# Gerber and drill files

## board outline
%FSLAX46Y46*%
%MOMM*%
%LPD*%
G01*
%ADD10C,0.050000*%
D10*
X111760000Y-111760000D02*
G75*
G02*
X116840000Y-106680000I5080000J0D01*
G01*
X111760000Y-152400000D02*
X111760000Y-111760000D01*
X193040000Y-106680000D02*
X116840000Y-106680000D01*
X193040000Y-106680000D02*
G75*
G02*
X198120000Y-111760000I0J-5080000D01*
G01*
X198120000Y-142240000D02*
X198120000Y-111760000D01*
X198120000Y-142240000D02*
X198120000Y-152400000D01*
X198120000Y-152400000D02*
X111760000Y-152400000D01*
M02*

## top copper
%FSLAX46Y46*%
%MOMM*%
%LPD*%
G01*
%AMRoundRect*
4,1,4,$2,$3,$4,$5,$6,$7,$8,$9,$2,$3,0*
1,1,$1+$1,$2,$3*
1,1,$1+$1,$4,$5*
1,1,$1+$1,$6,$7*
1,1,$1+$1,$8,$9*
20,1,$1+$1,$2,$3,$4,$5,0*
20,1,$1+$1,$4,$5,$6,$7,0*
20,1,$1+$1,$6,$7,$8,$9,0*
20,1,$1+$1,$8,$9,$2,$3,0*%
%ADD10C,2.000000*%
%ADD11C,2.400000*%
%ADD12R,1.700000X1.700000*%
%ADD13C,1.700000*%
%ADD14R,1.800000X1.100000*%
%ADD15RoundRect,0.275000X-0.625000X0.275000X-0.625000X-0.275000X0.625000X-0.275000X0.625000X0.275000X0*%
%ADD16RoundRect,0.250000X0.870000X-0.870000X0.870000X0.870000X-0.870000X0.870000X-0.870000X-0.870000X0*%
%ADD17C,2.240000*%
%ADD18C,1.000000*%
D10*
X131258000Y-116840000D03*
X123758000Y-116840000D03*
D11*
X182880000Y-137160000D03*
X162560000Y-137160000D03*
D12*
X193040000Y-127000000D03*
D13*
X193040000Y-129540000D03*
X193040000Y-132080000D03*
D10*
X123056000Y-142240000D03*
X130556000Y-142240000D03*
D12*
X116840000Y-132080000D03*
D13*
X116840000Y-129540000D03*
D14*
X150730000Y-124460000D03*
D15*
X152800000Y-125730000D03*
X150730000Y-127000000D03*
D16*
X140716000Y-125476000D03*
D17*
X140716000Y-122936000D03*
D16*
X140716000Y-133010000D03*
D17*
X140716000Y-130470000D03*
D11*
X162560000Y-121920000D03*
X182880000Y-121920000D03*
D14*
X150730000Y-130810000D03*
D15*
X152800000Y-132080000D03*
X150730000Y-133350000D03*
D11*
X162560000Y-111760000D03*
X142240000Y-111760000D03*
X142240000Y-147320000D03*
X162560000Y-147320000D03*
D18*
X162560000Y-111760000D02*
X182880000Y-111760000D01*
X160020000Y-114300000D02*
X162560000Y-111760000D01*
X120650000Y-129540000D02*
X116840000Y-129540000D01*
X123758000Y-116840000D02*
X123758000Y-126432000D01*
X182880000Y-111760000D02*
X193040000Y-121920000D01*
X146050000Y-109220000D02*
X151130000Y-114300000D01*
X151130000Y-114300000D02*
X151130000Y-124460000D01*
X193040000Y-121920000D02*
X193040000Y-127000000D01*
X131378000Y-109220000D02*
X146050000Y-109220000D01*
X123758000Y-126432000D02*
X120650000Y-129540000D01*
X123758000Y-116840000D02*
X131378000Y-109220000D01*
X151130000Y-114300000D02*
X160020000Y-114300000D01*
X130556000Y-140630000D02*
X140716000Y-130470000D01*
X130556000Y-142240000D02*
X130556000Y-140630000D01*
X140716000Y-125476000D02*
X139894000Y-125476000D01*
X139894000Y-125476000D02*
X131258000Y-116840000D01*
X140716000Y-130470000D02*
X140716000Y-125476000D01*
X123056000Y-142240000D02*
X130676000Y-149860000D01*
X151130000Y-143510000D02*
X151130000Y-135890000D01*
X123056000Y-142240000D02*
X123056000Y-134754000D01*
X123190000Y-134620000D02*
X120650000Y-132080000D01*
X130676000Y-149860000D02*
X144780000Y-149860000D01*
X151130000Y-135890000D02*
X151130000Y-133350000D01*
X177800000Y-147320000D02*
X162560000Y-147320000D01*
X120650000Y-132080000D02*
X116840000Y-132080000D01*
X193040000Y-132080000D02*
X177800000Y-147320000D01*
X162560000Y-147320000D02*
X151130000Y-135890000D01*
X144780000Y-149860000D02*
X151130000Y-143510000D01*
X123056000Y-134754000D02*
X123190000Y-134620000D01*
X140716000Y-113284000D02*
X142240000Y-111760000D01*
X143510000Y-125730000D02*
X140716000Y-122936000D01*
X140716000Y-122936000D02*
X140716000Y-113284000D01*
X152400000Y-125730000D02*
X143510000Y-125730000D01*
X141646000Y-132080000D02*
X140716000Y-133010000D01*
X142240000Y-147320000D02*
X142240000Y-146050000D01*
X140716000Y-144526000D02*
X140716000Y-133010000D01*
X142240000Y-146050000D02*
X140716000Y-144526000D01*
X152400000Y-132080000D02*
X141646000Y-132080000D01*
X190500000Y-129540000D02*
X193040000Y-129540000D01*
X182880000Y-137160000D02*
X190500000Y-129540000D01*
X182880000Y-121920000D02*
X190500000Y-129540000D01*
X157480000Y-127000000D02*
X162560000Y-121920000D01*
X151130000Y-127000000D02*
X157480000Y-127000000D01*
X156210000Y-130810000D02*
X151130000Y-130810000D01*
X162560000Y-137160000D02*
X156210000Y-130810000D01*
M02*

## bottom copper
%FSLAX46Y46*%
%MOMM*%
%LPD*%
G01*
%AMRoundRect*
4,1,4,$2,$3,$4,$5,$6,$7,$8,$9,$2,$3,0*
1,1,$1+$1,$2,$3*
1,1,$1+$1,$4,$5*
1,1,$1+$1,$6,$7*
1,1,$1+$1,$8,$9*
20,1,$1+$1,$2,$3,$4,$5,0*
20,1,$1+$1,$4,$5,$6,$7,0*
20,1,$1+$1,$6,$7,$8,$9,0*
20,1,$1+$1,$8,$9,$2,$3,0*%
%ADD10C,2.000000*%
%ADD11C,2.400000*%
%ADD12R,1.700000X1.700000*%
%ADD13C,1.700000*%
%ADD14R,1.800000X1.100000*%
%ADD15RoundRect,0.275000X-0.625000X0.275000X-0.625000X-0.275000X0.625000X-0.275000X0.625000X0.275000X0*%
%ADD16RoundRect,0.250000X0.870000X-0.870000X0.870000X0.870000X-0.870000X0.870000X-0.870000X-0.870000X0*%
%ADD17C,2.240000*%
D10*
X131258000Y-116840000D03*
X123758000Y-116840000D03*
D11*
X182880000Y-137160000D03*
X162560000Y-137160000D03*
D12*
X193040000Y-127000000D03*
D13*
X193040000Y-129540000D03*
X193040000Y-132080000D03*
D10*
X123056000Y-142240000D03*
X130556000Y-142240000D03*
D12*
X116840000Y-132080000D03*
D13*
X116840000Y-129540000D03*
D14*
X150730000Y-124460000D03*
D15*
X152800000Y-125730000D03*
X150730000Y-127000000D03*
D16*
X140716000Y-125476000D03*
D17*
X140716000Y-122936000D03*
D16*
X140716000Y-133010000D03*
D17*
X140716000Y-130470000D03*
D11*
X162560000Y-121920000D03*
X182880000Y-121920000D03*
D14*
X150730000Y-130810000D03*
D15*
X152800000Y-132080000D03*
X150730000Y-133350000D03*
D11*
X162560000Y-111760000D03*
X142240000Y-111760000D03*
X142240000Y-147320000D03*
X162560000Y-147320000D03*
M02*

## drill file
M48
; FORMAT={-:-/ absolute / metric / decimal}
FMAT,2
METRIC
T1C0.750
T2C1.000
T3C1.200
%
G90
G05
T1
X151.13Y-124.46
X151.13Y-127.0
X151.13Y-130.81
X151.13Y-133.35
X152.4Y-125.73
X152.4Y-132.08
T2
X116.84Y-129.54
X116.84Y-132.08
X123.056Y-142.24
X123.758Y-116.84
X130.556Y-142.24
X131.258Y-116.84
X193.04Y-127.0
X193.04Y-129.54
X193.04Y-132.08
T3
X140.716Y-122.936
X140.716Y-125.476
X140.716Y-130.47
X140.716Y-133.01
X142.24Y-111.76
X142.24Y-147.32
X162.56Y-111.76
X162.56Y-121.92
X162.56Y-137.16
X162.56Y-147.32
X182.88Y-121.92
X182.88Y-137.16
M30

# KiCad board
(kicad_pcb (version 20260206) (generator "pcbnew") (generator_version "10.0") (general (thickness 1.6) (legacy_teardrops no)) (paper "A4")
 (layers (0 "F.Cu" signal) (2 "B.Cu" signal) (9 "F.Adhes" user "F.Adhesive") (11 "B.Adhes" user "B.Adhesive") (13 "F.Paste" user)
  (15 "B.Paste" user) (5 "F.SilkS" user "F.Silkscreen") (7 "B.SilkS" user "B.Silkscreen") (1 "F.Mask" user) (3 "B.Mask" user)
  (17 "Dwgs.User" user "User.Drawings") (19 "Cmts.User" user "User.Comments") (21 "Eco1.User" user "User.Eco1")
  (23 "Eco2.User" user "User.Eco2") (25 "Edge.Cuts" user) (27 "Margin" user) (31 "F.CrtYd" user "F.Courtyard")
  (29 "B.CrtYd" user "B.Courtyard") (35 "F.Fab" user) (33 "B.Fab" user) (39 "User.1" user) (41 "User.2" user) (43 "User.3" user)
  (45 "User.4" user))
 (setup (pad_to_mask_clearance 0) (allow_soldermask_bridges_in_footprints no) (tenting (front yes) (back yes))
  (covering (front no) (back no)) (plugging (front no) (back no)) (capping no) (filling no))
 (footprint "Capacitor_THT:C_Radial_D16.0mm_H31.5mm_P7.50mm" (layer "F.Cu") (at 131.258 116.84 180)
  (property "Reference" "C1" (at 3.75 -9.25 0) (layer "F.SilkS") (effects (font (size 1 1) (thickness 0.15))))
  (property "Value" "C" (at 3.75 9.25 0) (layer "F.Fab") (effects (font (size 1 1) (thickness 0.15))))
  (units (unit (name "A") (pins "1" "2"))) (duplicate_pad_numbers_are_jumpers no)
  (pad "1" thru_hole circle (at 0 0 180) (size 2 2) (drill 1) (layers "*.Cu" "*.Mask") (remove_unused_layers no) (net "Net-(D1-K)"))
  (pad "2" thru_hole circle (at 7.5 0 180) (size 2 2) (drill 1) (layers "*.Cu" "*.Mask") (remove_unused_layers no) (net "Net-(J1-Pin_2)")))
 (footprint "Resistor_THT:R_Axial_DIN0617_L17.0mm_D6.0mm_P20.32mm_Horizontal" (layer "F.Cu") (at 182.88 137.16 180)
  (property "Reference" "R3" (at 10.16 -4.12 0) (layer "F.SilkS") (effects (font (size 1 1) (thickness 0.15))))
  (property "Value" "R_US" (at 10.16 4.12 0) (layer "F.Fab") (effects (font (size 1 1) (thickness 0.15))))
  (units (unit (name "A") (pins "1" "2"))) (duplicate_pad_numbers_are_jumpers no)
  (pad "1" thru_hole circle (at 0 0 180) (size 2.4 2.4) (drill 1.2) (layers "*.Cu" "*.Mask") (remove_unused_layers no)
   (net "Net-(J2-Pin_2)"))
  (pad "2" thru_hole circle (at 20.32 0 180) (size 2.4 2.4) (drill 1.2) (layers "*.Cu" "*.Mask") (remove_unused_layers no)
   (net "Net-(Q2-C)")))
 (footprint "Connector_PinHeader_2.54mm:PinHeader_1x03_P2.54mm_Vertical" (layer "F.Cu") (at 193.04 127)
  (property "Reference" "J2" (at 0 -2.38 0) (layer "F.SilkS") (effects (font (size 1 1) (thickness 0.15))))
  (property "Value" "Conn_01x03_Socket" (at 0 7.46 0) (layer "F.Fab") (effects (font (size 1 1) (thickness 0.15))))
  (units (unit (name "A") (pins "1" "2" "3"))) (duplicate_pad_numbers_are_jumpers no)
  (pad "1" thru_hole rect (at 0 0) (size 1.7 1.7) (drill 1) (layers "*.Cu" "*.Mask") (remove_unused_layers no) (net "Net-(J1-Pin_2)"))
  (pad "2" thru_hole circle (at 0 2.54) (size 1.7 1.7) (drill 1) (layers "*.Cu" "*.Mask") (remove_unused_layers no) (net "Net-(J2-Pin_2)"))
  (pad "3" thru_hole circle (at 0 5.08) (size 1.7 1.7) (drill 1) (layers "*.Cu" "*.Mask") (remove_unused_layers no) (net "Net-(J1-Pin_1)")))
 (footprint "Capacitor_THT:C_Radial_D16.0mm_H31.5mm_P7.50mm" (layer "F.Cu") (at 123.056 142.24)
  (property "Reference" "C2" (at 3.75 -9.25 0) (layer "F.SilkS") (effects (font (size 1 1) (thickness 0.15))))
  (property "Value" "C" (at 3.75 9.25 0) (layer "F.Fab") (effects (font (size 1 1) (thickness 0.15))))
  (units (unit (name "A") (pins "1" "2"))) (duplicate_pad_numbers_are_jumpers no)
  (pad "1" thru_hole circle (at 0 0) (size 2 2) (drill 1) (layers "*.Cu" "*.Mask") (remove_unused_layers no) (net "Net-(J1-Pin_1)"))
  (pad "2" thru_hole circle (at 7.5 0) (size 2 2) (drill 1) (layers "*.Cu" "*.Mask") (remove_unused_layers no) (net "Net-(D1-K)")))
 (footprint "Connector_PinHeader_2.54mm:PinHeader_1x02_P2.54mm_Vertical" (layer "F.Cu") (at 116.84 132.08 180)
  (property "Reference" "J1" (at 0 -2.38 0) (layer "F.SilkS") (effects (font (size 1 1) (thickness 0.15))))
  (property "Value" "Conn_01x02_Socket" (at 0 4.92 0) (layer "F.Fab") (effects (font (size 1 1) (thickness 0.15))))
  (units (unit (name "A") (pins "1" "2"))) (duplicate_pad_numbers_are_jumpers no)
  (pad "1" thru_hole rect (at 0 0 180) (size 1.7 1.7) (drill 1) (layers "*.Cu" "*.Mask") (remove_unused_layers no) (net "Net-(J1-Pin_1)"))
  (pad "2" thru_hole circle (at 0 2.54 180) (size 1.7 1.7) (drill 1) (layers "*.Cu" "*.Mask") (remove_unused_layers no)
   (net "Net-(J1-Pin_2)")))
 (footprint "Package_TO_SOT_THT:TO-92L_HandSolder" (layer "F.Cu") (at 151.13 124.46 -90)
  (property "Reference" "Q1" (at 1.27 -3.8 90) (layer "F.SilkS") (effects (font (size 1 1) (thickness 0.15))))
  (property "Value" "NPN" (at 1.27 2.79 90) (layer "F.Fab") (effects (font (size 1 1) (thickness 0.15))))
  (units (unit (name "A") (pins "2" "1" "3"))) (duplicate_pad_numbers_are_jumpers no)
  (pad "1" thru_hole rect (at 0 0 270) (size 1.1 1.8) (drill 0.75 (offset 0 0.4)) (layers "*.Cu" "*.Mask") (remove_unused_layers no)
   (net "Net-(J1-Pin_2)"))
  (pad "2" thru_hole roundrect (at 1.27 -1.27 270) (size 1.1 1.8) (drill 0.75 (offset 0 -0.4)) (layers "*.Cu" "*.Mask")
   (remove_unused_layers no) (roundrect_rratio 0.25) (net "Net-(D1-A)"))
  (pad "3" thru_hole roundrect (at 2.54 0 270) (size 1.1 1.8) (drill 0.75 (offset 0 0.4)) (layers "*.Cu" "*.Mask") (remove_unused_layers no)
   (roundrect_rratio 0.25) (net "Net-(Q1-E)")))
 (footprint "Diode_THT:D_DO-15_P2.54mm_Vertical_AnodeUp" (layer "F.Cu") (at 140.716 125.476 90)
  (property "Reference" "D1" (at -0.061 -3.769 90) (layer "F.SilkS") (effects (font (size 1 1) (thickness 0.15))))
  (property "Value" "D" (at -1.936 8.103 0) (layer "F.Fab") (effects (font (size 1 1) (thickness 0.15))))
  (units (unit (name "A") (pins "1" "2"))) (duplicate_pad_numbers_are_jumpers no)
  (pad "1" thru_hole roundrect (at 0 0 90) (size 2.24 2.24) (drill 1.2) (layers "*.Cu" "*.Mask") (remove_unused_layers no)
   (roundrect_rratio 0.111607) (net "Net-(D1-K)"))
  (pad "2" thru_hole circle (at 2.54 0 90) (size 2.24 2.24) (drill 1.2) (layers "*.Cu" "*.Mask") (remove_unused_layers no)
   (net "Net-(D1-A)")))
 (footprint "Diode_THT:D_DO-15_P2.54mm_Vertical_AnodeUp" (layer "F.Cu") (at 140.716 133.01 90)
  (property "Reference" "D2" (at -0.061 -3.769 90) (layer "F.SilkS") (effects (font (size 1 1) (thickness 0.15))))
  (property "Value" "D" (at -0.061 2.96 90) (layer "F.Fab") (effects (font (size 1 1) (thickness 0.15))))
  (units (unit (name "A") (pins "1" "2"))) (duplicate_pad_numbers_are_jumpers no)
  (pad "1" thru_hole roundrect (at 0 0 90) (size 2.24 2.24) (drill 1.2) (layers "*.Cu" "*.Mask") (remove_unused_layers no)
   (roundrect_rratio 0.111607) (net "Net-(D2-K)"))
  (pad "2" thru_hole circle (at 2.54 0 90) (size 2.24 2.24) (drill 1.2) (layers "*.Cu" "*.Mask") (remove_unused_layers no)
   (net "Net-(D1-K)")))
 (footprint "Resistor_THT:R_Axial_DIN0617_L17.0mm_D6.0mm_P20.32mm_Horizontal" (layer "F.Cu") (at 162.56 121.92)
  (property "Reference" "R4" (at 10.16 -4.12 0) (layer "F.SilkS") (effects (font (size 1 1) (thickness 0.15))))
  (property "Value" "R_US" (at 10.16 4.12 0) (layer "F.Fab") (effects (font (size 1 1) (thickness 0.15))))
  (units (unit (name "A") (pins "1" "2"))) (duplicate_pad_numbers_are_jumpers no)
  (pad "1" thru_hole circle (at 0 0) (size 2.4 2.4) (drill 1.2) (layers "*.Cu" "*.Mask") (remove_unused_layers no) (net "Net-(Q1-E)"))
  (pad "2" thru_hole circle (at 20.32 0) (size 2.4 2.4) (drill 1.2) (layers "*.Cu" "*.Mask") (remove_unused_layers no)
   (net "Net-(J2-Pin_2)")))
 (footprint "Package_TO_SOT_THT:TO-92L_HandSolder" (layer "F.Cu") (at 151.13 130.81 -90)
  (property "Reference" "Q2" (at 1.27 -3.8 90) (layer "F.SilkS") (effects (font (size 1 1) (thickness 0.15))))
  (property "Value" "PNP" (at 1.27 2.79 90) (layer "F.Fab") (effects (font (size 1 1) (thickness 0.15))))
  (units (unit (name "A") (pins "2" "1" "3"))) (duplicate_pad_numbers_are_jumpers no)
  (pad "1" thru_hole rect (at 0 0 270) (size 1.1 1.8) (drill 0.75 (offset 0 0.4)) (layers "*.Cu" "*.Mask") (remove_unused_layers no)
   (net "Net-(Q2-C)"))
  (pad "2" thru_hole roundrect (at 1.27 -1.27 270) (size 1.1 1.8) (drill 0.75 (offset 0 -0.4)) (layers "*.Cu" "*.Mask")
   (remove_unused_layers no) (roundrect_rratio 0.25) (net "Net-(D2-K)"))
  (pad "3" thru_hole roundrect (at 2.54 0 270) (size 1.1 1.8) (drill 0.75 (offset 0 0.4)) (layers "*.Cu" "*.Mask") (remove_unused_layers no)
   (roundrect_rratio 0.25) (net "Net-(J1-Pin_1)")))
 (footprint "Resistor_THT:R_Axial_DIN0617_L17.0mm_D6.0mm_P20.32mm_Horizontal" (layer "F.Cu") (at 162.56 111.76 180)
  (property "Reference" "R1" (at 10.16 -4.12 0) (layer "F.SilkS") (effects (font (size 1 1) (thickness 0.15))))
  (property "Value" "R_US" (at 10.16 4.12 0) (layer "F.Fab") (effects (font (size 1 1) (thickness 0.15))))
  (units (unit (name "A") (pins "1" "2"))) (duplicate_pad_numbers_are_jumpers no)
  (pad "1" thru_hole circle (at 0 0 180) (size 2.4 2.4) (drill 1.2) (layers "*.Cu" "*.Mask") (remove_unused_layers no)
   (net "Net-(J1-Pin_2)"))
  (pad "2" thru_hole circle (at 20.32 0 180) (size 2.4 2.4) (drill 1.2) (layers "*.Cu" "*.Mask") (remove_unused_layers no)
   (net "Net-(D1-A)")))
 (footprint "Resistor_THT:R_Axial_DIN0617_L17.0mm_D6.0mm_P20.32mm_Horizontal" (layer "F.Cu") (at 142.24 147.32)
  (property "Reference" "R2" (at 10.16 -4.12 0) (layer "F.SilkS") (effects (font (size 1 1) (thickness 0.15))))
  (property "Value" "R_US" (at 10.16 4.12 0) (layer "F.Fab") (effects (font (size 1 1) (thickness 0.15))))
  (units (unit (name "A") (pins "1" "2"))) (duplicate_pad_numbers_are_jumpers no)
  (pad "1" thru_hole circle (at 0 0) (size 2.4 2.4) (drill 1.2) (layers "*.Cu" "*.Mask") (remove_unused_layers no) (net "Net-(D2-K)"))
  (pad "2" thru_hole circle (at 20.32 0) (size 2.4 2.4) (drill 1.2) (layers "*.Cu" "*.Mask") (remove_unused_layers no)
   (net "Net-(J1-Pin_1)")))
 (gr_arc (start 111.76 111.76) (mid 113.247898 108.167898) (end 116.84 106.68) (stroke (width 0.05) (type default)) (layer "Edge.Cuts"))
 (gr_line (start 111.76 152.4) (end 111.76 111.76) (stroke (width 0.05) (type default)) (layer "Edge.Cuts"))
 (gr_line (start 193.04 106.68) (end 116.84 106.68) (stroke (width 0.05) (type default)) (layer "Edge.Cuts"))
 (gr_arc (start 193.04 106.68) (mid 196.632102 108.167898) (end 198.12 111.76) (stroke (width 0.05) (type default)) (layer "Edge.Cuts"))
 (gr_line (start 198.12 142.24) (end 198.12 111.76) (stroke (width 0.05) (type default)) (layer "Edge.Cuts"))
 (gr_line (start 198.12 142.24) (end 198.12 152.4) (stroke (width 0.05) (type default)) (layer "Edge.Cuts"))
 (gr_line (start 198.12 152.4) (end 111.76 152.4) (stroke (width 0.05) (type default)) (layer "Edge.Cuts"))
 (segment (start 162.56 111.76) (end 182.88 111.76) (width 1) (layer "F.Cu") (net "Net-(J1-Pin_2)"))
 (segment (start 160.02 114.3) (end 162.56 111.76) (width 1) (layer "F.Cu") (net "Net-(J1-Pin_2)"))
 (segment (start 120.65 129.54) (end 116.84 129.54) (width 1) (layer "F.Cu") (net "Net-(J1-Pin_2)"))
 (segment (start 123.758 116.84) (end 123.758 126.432) (width 1) (layer "F.Cu") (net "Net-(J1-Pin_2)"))
 (segment (start 182.88 111.76) (end 193.04 121.92) (width 1) (layer "F.Cu") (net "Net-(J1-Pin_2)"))
 (segment (start 146.05 109.22) (end 151.13 114.3) (width 1) (layer "F.Cu") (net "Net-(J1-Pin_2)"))
 (segment (start 151.13 114.3) (end 151.13 124.46) (width 1) (layer "F.Cu") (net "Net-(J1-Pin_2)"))
 (segment (start 193.04 121.92) (end 193.04 127) (width 1) (layer "F.Cu") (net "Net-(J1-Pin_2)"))
 (segment (start 131.378 109.22) (end 146.05 109.22) (width 1) (layer "F.Cu") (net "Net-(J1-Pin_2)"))
 (segment (start 123.758 126.432) (end 120.65 129.54) (width 1) (layer "F.Cu") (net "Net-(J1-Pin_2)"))
 (segment (start 123.758 116.84) (end 131.378 109.22) (width 1) (layer "F.Cu") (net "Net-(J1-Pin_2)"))
 (segment (start 151.13 114.3) (end 160.02 114.3) (width 1) (layer "F.Cu") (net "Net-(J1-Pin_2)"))
 (segment (start 130.556 140.63) (end 140.716 130.47) (width 1) (layer "F.Cu") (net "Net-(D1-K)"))
 (segment (start 130.556 142.24) (end 130.556 140.63) (width 1) (layer "F.Cu") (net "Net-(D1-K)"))
 (segment (start 140.716 125.476) (end 139.894 125.476) (width 1) (layer "F.Cu") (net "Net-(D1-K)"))
 (segment (start 139.894 125.476) (end 131.258 116.84) (width 1) (layer "F.Cu") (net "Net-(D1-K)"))
 (segment (start 140.716 130.47) (end 140.716 125.476) (width 1) (layer "F.Cu") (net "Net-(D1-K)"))
 (segment (start 123.056 142.24) (end 130.676 149.86) (width 1) (layer "F.Cu") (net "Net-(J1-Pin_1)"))
 (segment (start 151.13 143.51) (end 151.13 135.89) (width 1) (layer "F.Cu") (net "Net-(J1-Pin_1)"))
 (segment (start 123.056 142.24) (end 123.056 134.754) (width 1) (layer "F.Cu") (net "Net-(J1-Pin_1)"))
 (segment (start 123.19 134.62) (end 120.65 132.08) (width 1) (layer "F.Cu") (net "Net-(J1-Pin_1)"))
 (segment (start 130.676 149.86) (end 144.78 149.86) (width 1) (layer "F.Cu") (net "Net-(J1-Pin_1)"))
 (segment (start 151.13 135.89) (end 151.13 133.35) (width 1) (layer "F.Cu") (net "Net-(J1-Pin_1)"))
 (segment (start 177.8 147.32) (end 162.56 147.32) (width 1) (layer "F.Cu") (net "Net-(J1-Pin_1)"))
 (segment (start 120.65 132.08) (end 116.84 132.08) (width 1) (layer "F.Cu") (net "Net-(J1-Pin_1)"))
 (segment (start 193.04 132.08) (end 177.8 147.32) (width 1) (layer "F.Cu") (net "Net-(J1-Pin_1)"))
 (segment (start 162.56 147.32) (end 151.13 135.89) (width 1) (layer "F.Cu") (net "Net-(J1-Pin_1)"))
 (segment (start 144.78 149.86) (end 151.13 143.51) (width 1) (layer "F.Cu") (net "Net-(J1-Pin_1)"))
 (segment (start 123.056 134.754) (end 123.19 134.62) (width 1) (layer "F.Cu") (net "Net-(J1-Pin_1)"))
 (segment (start 140.716 113.284) (end 142.24 111.76) (width 1) (layer "F.Cu") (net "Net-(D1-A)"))
 (segment (start 143.51 125.73) (end 140.716 122.936) (width 1) (layer "F.Cu") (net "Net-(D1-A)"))
 (segment (start 140.716 122.936) (end 140.716 113.284) (width 1) (layer "F.Cu") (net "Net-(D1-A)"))
 (segment (start 152.4 125.73) (end 143.51 125.73) (width 1) (layer "F.Cu") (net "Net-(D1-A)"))
 (segment (start 141.646 132.08) (end 140.716 133.01) (width 1) (layer "F.Cu") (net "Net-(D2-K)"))
 (segment (start 142.24 147.32) (end 142.24 146.05) (width 1) (layer "F.Cu") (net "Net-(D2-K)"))
 (segment (start 140.716 144.526) (end 140.716 133.01) (width 1) (layer "F.Cu") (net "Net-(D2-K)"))
 (segment (start 142.24 146.05) (end 140.716 144.526) (width 1) (layer "F.Cu") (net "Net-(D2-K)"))
 (segment (start 152.4 132.08) (end 141.646 132.08) (width 1) (layer "F.Cu") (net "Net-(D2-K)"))
 (segment (start 190.5 129.54) (end 193.04 129.54) (width 1) (layer "F.Cu") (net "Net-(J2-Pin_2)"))
 (segment (start 182.88 137.16) (end 190.5 129.54) (width 1) (layer "F.Cu") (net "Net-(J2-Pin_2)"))
 (segment (start 182.88 121.92) (end 190.5 129.54) (width 1) (layer "F.Cu") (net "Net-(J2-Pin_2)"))
 (segment (start 157.48 127) (end 162.56 121.92) (width 1) (layer "F.Cu") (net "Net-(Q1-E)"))
 (segment (start 151.13 127) (end 157.48 127) (width 1) (layer "F.Cu") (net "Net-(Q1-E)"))
 (segment (start 156.21 130.81) (end 151.13 130.81) (width 1) (layer "F.Cu") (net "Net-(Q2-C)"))
 (segment (start 162.56 137.16) (end 156.21 130.81) (width 1) (layer "F.Cu") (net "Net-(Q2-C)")))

